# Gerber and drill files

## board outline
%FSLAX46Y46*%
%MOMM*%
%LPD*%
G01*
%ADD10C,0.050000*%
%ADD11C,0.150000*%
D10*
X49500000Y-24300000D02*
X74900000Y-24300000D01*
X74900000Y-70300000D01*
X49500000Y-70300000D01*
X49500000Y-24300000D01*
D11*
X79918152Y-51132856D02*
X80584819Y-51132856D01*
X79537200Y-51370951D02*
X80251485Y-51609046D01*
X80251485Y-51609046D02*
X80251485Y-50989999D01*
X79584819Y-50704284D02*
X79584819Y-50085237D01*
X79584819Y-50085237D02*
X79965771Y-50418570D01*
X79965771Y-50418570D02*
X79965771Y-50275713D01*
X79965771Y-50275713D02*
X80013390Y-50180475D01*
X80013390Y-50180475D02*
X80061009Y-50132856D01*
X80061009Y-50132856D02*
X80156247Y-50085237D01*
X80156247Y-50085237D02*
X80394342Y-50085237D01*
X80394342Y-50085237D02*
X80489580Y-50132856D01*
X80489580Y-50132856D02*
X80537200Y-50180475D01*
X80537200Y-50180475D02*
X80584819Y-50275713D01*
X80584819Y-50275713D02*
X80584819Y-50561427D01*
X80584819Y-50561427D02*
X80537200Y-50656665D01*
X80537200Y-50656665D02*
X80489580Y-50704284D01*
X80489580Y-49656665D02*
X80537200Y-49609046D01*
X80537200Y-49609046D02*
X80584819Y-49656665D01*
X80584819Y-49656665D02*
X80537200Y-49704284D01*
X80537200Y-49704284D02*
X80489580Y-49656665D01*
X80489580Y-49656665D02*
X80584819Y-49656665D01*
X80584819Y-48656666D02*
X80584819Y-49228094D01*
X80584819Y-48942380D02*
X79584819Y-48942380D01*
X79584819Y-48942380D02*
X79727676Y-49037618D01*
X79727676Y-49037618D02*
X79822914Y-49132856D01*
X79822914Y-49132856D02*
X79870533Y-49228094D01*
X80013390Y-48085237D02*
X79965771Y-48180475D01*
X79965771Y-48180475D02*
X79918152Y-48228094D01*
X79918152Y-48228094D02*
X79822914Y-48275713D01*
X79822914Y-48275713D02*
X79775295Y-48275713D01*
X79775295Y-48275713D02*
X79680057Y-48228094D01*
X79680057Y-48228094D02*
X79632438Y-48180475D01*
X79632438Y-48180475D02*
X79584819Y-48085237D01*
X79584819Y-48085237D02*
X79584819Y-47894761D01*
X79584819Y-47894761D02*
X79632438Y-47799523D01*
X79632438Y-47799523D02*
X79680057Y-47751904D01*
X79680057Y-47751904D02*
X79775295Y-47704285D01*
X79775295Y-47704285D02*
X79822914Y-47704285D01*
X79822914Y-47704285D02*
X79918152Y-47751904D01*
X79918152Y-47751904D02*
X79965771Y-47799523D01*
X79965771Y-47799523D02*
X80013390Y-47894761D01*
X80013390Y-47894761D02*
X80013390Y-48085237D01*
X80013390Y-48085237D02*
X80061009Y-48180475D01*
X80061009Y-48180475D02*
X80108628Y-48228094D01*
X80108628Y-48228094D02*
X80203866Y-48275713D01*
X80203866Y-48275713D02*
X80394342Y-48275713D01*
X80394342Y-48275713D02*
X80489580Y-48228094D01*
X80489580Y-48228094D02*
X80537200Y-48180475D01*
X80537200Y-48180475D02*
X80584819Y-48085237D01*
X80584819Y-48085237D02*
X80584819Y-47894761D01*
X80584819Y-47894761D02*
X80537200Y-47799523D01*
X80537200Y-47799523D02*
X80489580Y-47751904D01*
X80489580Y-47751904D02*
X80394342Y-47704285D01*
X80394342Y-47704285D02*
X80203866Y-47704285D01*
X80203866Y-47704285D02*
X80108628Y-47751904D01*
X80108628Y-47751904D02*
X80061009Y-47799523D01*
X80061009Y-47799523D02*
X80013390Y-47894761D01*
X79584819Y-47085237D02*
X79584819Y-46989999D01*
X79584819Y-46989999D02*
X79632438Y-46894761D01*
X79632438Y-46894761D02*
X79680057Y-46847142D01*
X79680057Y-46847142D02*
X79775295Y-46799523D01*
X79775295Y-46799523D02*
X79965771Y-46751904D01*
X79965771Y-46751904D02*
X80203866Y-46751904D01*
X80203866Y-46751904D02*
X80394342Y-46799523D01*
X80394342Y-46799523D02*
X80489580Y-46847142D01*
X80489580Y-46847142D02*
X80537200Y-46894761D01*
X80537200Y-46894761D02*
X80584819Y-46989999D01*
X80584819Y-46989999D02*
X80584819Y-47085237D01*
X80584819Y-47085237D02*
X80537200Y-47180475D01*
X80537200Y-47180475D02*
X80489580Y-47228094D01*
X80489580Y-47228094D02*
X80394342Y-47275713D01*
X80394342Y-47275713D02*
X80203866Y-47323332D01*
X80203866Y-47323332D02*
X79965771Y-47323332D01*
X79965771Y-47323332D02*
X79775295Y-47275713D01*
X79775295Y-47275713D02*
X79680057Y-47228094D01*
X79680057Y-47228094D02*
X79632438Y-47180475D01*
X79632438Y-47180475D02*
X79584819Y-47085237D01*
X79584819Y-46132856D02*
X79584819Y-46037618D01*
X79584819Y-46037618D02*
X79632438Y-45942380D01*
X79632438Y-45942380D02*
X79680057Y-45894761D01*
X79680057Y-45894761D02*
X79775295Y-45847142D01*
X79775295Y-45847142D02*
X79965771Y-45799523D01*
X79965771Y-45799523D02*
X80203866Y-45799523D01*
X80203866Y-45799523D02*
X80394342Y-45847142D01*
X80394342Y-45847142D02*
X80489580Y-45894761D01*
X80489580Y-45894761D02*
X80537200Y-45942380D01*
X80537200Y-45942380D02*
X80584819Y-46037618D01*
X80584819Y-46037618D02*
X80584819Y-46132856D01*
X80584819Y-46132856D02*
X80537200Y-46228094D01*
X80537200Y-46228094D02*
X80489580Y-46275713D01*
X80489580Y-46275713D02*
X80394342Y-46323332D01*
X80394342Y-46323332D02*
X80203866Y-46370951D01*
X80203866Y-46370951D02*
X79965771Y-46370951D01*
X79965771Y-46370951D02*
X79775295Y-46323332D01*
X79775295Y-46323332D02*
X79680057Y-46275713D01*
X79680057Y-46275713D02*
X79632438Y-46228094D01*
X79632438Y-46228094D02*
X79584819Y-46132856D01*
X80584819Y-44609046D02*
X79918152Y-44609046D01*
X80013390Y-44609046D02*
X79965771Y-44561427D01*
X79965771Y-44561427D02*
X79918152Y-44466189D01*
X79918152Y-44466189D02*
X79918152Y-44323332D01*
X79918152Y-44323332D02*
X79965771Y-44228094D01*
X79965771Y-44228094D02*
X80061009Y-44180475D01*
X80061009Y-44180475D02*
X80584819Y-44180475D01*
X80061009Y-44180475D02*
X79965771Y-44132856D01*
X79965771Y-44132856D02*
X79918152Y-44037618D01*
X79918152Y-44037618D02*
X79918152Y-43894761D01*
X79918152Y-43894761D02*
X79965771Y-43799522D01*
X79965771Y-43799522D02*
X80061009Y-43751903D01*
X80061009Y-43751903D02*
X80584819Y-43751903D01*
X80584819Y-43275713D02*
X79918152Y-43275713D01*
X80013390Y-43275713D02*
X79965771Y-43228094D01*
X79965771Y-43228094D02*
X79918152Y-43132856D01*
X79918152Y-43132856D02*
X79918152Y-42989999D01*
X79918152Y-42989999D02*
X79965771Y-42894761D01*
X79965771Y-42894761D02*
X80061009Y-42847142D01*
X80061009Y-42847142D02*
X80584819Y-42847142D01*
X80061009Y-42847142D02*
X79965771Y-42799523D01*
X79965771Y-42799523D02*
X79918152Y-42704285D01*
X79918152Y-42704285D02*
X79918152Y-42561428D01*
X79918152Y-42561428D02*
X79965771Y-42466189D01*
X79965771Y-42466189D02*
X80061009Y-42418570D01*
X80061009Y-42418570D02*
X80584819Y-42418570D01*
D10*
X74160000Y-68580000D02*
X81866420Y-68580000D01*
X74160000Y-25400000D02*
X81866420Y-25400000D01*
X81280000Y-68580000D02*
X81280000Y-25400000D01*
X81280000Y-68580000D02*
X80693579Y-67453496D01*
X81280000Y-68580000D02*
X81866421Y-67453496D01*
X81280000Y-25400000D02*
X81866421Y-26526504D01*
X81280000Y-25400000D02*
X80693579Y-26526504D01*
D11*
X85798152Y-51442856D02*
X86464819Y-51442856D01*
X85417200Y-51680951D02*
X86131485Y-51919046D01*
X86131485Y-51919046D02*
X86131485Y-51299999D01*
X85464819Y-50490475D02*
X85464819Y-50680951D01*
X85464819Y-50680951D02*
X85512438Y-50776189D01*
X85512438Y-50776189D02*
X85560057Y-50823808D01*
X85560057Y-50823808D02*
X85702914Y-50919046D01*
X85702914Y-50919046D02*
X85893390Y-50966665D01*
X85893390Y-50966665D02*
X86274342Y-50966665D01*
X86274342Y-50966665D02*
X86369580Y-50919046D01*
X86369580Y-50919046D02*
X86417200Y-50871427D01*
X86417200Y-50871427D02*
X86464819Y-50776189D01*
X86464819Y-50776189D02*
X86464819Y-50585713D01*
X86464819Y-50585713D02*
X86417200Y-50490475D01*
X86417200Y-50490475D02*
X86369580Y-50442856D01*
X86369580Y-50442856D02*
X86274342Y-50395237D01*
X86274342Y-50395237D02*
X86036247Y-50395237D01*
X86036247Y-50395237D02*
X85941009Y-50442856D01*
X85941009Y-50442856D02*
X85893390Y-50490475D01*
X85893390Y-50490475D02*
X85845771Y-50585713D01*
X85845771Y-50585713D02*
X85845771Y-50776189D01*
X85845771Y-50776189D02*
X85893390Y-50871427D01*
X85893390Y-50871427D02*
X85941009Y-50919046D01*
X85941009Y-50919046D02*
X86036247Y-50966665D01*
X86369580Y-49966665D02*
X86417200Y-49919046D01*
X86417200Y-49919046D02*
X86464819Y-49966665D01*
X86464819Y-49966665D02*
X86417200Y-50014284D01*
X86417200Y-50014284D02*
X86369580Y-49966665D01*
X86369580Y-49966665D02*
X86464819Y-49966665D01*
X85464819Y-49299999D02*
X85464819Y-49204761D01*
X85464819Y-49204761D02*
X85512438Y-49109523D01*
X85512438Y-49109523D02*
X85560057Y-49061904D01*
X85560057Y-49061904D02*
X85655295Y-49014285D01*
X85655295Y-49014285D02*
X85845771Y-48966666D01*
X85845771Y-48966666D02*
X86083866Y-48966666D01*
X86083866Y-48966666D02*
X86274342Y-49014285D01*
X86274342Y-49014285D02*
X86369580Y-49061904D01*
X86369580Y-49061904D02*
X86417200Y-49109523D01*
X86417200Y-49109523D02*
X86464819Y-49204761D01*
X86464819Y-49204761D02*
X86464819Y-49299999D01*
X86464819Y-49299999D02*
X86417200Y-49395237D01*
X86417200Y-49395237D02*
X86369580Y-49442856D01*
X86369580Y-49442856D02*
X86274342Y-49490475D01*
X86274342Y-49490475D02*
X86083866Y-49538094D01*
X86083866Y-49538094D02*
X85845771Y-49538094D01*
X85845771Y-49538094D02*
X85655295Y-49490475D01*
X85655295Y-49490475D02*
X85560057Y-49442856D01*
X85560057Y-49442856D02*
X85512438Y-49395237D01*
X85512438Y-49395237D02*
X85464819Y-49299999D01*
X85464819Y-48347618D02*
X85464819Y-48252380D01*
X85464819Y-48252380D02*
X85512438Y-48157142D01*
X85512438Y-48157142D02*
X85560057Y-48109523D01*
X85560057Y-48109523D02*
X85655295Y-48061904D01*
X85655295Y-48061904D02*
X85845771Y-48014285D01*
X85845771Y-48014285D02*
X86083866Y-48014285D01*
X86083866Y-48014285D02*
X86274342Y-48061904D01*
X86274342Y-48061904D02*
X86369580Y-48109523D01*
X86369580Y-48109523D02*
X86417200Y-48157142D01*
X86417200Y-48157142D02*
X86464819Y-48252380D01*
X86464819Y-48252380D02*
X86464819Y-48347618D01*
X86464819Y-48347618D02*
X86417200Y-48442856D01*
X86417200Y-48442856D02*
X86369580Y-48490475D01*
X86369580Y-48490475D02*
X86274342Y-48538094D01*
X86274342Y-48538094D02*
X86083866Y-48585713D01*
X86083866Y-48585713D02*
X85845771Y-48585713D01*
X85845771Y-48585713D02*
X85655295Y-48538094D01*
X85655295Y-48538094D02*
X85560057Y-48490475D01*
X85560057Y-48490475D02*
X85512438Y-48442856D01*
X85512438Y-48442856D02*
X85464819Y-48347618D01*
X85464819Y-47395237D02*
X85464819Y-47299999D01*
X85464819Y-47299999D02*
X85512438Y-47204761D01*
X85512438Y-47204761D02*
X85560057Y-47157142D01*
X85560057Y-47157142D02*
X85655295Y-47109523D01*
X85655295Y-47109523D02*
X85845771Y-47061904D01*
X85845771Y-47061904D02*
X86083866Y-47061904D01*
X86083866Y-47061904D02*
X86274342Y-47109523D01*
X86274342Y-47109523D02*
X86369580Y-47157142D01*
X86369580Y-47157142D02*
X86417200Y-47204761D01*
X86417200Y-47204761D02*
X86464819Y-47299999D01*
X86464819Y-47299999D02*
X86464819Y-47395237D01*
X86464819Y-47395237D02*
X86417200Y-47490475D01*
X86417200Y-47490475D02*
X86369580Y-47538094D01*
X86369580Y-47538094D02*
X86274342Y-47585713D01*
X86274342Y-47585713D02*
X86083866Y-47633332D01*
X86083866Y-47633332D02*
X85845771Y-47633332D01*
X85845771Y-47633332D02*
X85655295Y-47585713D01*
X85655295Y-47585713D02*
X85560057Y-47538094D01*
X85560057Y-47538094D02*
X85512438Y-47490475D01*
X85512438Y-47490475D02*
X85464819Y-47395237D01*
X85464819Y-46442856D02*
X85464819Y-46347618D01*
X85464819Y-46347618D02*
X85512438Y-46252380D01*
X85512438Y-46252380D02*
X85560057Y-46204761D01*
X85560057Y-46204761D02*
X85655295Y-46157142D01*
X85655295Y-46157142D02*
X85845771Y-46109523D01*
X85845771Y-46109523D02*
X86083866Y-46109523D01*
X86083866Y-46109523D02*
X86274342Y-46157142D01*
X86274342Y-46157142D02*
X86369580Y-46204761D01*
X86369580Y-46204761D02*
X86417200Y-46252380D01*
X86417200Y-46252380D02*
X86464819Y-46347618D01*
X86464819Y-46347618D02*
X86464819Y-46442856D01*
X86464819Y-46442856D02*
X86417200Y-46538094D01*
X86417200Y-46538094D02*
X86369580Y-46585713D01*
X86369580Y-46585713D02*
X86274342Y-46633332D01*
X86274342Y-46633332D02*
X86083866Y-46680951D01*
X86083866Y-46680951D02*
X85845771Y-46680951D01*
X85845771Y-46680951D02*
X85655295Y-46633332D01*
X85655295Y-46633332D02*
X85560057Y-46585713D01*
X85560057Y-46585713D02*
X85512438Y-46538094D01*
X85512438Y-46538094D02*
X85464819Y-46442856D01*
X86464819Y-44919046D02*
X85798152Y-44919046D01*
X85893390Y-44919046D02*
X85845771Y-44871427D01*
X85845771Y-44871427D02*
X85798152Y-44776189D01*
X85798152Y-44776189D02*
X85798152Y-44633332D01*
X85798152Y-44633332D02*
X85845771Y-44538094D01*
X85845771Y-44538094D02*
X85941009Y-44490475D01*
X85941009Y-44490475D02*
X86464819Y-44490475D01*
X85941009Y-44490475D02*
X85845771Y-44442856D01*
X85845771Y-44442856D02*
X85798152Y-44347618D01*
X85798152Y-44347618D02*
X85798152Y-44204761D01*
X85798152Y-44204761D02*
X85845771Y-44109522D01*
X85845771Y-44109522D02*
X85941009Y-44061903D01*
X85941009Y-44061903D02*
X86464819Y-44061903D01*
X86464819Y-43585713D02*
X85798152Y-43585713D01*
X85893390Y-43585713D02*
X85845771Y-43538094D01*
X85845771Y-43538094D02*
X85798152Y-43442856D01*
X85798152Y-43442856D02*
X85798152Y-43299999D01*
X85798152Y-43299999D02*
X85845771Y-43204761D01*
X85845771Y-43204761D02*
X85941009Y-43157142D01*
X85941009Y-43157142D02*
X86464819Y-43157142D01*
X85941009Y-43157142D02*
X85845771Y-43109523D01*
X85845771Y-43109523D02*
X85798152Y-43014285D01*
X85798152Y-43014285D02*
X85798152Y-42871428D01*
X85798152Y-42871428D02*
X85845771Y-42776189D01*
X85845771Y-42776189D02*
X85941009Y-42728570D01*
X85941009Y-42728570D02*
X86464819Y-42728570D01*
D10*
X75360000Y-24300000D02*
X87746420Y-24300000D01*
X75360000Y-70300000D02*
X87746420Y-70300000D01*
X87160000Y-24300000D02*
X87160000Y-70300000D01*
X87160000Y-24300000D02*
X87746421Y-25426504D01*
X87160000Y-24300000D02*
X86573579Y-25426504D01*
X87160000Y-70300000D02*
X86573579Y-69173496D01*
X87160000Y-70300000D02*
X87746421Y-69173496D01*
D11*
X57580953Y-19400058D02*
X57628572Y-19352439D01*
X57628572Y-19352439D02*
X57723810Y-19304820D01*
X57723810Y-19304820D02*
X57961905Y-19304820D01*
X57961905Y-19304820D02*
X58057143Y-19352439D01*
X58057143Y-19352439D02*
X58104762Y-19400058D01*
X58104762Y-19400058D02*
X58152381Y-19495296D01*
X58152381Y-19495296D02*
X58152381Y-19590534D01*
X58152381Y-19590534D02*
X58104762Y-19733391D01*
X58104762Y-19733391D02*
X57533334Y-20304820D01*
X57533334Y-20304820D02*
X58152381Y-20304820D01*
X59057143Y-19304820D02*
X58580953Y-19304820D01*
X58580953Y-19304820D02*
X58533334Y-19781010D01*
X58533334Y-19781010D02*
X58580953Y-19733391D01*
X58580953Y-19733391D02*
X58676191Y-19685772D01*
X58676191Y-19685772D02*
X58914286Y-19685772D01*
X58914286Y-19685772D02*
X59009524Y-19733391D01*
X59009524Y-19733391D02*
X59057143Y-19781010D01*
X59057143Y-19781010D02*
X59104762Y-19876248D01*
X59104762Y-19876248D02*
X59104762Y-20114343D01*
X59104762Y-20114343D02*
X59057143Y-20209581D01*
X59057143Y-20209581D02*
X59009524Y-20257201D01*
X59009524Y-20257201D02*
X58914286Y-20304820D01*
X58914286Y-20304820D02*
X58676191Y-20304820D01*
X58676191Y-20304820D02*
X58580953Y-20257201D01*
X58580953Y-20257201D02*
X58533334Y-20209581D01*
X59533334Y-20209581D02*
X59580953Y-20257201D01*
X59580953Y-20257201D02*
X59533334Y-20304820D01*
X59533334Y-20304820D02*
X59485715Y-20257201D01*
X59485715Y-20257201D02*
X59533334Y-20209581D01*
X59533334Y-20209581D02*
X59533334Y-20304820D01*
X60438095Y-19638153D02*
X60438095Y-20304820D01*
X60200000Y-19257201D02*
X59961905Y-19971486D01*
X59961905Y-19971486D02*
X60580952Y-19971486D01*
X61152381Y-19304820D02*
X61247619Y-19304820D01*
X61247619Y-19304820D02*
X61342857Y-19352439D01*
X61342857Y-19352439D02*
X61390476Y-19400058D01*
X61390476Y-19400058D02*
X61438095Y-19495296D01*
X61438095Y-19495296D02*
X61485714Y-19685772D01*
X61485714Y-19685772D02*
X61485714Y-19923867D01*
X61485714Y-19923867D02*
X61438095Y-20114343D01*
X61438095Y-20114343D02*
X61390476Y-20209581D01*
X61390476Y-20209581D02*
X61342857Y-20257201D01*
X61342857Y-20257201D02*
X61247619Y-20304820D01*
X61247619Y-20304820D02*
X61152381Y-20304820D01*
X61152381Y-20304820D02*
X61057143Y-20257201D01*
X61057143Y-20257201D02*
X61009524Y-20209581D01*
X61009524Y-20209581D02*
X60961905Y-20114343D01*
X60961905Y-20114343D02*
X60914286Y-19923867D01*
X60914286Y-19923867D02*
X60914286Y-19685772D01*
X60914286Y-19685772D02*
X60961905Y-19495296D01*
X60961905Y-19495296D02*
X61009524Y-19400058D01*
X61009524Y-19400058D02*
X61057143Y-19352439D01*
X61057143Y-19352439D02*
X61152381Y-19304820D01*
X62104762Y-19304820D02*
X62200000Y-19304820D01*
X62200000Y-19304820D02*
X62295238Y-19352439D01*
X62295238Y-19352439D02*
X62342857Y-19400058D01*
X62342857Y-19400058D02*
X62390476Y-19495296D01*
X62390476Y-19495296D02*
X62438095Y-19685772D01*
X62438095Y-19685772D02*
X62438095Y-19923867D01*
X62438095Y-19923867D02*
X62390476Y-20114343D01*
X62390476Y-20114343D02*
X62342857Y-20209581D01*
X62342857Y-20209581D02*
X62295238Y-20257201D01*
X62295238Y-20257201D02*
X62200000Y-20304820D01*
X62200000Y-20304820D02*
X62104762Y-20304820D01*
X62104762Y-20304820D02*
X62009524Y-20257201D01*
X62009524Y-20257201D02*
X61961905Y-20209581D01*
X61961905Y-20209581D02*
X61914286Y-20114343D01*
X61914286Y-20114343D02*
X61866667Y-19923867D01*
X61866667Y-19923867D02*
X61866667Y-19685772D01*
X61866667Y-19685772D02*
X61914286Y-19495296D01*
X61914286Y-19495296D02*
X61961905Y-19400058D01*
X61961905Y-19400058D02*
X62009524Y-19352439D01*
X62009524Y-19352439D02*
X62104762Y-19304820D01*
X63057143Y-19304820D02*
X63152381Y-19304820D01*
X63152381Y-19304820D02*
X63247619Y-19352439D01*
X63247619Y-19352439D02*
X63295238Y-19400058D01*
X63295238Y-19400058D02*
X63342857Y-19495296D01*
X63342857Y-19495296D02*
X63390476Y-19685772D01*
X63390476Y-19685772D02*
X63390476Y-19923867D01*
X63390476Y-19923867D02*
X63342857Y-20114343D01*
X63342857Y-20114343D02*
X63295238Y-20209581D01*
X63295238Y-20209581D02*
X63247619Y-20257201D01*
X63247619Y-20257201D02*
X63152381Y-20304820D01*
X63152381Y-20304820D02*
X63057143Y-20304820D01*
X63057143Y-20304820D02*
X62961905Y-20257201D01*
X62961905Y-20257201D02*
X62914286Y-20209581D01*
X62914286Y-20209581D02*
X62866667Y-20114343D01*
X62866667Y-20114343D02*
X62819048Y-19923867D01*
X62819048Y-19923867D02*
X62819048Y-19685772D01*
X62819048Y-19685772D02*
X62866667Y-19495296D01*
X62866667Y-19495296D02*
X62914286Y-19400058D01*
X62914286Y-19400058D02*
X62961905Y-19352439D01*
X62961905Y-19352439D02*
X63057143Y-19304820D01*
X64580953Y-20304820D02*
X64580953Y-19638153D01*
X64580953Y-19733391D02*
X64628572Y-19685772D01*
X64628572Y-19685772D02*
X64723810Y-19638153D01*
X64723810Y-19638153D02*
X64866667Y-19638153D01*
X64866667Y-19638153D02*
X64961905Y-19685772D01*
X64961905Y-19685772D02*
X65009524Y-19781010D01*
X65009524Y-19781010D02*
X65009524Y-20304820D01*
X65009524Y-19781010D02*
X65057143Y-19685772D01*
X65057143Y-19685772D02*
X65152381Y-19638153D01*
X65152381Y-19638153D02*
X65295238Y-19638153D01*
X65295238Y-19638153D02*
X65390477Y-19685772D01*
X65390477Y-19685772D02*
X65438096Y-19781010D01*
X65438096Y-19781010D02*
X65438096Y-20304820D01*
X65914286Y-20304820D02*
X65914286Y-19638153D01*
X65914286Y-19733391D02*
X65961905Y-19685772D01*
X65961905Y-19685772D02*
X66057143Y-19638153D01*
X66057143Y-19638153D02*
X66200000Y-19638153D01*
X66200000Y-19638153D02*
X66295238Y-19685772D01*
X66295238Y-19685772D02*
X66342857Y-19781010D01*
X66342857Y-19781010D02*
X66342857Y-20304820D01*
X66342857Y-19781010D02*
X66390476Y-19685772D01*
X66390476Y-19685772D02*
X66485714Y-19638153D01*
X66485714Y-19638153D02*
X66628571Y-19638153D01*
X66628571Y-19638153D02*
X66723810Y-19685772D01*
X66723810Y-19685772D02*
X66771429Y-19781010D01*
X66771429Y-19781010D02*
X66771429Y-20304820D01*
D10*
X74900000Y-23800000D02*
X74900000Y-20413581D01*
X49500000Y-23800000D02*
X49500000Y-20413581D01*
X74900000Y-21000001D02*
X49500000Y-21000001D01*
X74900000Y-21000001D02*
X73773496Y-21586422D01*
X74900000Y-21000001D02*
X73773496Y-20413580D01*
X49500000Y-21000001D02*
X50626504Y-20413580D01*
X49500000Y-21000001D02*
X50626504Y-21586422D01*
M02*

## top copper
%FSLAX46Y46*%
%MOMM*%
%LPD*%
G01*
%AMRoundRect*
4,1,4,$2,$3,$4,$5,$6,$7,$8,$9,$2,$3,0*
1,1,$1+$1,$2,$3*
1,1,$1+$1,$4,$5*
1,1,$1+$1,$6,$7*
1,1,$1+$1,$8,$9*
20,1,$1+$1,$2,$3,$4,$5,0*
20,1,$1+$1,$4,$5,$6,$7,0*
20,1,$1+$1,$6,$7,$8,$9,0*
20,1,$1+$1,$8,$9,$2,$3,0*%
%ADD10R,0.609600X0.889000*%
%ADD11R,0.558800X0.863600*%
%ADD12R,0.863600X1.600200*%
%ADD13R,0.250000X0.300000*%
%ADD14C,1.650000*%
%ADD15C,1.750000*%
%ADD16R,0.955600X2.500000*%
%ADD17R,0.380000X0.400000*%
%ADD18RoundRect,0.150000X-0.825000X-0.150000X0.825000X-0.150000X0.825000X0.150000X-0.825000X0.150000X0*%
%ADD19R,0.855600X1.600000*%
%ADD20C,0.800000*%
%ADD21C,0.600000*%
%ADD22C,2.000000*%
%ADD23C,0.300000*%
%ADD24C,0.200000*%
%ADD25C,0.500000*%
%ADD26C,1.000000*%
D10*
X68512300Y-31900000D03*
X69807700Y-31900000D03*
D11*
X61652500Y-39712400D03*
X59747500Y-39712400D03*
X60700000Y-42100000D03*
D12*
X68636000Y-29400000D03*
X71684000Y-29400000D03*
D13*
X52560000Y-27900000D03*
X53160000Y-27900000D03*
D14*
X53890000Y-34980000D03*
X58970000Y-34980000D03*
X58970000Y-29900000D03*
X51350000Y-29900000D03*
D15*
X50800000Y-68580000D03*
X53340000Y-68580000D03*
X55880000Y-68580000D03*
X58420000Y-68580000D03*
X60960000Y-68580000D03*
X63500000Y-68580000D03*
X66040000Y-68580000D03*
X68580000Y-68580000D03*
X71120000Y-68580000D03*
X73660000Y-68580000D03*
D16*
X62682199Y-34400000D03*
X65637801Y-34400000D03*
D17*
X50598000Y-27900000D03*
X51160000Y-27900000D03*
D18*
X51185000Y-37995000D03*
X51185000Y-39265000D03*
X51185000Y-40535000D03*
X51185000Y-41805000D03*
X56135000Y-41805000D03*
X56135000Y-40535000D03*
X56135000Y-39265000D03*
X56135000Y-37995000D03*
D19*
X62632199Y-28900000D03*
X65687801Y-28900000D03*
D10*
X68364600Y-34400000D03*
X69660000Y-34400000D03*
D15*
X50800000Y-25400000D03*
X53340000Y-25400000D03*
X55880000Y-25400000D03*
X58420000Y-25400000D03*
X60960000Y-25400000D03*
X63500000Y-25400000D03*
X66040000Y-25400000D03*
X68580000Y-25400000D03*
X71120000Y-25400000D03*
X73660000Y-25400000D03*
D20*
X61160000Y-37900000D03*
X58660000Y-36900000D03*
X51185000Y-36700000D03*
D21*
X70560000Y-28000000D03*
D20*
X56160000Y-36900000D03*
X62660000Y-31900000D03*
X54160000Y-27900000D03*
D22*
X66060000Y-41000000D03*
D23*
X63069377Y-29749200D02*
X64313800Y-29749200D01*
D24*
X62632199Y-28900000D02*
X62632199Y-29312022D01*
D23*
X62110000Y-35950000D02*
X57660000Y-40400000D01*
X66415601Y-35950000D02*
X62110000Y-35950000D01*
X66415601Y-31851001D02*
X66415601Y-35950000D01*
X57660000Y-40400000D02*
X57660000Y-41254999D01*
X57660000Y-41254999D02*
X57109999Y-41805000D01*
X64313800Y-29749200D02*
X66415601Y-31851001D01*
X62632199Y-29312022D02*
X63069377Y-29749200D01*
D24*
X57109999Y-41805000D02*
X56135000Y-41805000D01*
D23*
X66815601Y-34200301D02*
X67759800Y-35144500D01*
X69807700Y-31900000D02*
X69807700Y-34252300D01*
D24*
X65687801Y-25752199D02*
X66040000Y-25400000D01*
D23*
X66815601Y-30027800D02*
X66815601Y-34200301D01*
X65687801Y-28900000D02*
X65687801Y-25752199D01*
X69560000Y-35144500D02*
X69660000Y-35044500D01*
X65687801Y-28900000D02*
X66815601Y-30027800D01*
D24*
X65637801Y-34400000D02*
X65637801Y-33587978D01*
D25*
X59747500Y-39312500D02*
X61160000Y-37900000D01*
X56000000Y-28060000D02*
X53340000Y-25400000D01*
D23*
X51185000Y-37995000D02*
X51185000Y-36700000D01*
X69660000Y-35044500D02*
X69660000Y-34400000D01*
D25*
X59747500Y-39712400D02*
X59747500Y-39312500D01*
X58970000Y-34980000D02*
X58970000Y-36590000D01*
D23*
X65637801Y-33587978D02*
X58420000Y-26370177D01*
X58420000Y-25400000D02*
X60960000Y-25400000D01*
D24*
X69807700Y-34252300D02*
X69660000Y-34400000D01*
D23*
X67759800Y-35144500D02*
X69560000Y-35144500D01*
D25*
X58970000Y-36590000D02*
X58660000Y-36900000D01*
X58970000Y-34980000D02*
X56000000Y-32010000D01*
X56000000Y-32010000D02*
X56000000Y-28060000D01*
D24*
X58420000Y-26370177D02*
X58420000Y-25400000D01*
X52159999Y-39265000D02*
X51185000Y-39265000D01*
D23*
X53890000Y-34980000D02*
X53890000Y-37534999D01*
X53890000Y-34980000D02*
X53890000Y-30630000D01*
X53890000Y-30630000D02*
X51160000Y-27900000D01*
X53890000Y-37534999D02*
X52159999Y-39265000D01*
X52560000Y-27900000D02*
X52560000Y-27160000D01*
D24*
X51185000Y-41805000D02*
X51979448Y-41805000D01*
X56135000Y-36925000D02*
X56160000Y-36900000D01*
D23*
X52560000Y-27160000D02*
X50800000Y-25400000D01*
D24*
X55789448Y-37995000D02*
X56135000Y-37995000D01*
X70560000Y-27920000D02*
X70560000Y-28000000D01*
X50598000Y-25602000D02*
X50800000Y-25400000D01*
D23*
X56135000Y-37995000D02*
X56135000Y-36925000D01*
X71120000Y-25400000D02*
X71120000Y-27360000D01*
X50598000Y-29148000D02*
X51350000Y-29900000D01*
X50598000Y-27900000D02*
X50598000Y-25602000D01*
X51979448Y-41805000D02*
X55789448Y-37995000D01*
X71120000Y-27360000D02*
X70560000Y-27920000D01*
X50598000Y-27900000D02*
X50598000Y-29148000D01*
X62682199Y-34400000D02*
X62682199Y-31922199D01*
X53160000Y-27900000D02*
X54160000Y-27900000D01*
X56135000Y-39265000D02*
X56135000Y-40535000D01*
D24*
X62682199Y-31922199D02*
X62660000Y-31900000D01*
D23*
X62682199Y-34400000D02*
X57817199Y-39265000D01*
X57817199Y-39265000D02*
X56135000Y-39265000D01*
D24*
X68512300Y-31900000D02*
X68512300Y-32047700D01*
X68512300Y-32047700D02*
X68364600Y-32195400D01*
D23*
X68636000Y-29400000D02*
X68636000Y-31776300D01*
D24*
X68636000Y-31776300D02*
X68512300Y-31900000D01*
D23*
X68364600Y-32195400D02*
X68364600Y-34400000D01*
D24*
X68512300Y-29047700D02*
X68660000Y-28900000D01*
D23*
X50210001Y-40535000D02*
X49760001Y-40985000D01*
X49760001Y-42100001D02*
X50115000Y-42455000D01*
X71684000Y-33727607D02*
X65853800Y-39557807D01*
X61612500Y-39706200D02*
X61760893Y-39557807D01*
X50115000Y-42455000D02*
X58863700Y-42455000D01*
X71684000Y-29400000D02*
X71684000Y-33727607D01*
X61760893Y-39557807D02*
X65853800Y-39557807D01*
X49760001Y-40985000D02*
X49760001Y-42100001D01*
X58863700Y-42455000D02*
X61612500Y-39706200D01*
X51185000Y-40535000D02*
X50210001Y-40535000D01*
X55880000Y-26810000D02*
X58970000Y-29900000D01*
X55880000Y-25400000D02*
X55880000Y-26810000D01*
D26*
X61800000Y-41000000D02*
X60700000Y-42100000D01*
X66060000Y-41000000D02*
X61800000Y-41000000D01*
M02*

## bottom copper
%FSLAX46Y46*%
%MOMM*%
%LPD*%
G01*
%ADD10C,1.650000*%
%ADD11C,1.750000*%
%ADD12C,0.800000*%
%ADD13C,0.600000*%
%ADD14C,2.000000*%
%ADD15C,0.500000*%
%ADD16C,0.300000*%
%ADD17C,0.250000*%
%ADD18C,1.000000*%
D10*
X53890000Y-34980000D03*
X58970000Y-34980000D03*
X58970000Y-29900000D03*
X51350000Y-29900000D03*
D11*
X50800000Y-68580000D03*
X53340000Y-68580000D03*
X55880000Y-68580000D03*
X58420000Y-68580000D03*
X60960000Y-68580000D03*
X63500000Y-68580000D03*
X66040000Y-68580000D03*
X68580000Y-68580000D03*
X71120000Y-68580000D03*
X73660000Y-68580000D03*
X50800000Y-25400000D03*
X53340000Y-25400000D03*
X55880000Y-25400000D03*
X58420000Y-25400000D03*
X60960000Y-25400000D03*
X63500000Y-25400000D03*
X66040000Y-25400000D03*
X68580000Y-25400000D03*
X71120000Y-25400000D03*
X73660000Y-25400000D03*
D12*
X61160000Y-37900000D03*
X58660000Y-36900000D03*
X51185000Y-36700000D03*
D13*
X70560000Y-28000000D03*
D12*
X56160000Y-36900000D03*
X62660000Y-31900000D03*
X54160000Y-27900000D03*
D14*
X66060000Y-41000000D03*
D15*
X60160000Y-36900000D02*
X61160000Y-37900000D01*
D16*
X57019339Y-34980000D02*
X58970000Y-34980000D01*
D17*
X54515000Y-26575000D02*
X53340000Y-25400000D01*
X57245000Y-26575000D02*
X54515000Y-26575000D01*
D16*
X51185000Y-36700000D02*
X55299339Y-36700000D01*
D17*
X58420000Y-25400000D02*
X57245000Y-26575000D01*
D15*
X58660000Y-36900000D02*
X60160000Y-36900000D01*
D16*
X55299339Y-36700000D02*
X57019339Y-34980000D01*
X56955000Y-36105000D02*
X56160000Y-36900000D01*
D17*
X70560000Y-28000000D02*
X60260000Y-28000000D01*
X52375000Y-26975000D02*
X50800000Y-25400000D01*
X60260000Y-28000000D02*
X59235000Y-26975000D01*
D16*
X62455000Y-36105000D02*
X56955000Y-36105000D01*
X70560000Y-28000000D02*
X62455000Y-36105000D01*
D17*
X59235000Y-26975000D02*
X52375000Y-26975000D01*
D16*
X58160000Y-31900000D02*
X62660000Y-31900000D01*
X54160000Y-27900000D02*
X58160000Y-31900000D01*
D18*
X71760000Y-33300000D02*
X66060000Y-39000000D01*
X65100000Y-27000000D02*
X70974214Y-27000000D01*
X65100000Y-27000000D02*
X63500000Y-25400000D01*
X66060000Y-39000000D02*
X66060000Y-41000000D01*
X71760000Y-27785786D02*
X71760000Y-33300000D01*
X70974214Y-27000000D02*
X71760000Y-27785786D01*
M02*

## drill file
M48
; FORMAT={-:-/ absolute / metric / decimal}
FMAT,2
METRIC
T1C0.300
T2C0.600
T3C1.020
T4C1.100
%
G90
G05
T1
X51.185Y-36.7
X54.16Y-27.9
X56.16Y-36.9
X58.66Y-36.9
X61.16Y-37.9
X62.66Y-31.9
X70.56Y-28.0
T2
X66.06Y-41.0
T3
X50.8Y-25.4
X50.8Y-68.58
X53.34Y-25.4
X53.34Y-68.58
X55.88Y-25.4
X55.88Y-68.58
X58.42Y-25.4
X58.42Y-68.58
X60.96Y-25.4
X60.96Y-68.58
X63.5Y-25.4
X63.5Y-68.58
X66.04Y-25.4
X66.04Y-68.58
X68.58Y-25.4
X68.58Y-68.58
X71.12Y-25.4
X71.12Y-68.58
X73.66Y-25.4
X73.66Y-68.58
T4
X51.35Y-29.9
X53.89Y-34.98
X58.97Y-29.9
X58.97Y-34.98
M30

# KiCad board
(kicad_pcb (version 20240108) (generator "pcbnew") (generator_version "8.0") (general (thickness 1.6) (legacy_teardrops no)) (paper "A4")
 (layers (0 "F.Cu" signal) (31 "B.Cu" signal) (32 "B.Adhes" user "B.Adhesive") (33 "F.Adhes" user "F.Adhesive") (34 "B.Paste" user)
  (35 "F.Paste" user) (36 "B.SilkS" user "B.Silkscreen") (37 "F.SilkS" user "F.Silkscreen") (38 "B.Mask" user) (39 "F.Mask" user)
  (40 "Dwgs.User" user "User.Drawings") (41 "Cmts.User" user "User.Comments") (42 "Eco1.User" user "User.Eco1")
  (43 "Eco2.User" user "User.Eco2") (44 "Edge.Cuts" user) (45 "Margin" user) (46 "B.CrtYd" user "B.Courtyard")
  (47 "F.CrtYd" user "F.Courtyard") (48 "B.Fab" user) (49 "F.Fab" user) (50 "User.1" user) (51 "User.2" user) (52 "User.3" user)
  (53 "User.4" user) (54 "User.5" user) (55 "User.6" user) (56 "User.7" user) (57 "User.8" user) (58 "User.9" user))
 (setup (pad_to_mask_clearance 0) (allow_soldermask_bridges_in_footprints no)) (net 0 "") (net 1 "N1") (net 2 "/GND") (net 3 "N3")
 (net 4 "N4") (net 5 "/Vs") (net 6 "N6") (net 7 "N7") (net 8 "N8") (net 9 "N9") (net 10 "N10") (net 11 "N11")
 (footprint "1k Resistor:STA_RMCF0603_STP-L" (layer "F.Cu") (at 69.16 31.9)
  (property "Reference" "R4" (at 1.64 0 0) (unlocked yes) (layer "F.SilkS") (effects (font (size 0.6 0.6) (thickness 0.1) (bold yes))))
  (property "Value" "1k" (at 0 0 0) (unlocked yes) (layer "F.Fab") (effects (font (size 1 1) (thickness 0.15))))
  (pad "1" smd rect (at -0.6477 0) (size 0.6096 0.889) (layers "F.Cu" "F.Paste" "F.Mask") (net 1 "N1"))
  (pad "2" smd rect (at 0.6477 0) (size 0.6096 0.889) (layers "F.Cu" "F.Paste" "F.Mask") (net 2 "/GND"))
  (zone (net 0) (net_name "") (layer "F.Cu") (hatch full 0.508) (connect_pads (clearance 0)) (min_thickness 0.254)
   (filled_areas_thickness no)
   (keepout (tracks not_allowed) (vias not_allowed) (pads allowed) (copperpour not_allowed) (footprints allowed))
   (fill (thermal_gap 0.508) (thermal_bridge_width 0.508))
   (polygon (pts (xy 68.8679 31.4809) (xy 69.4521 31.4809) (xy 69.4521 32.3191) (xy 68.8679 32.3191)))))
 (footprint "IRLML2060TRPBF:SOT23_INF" (layer "F.Cu") (at 60.7 40.9062 180)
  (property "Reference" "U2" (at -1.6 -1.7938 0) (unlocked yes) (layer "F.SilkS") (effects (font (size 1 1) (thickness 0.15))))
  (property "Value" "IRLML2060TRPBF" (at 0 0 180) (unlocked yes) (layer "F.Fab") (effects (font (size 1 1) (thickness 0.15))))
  (pad "1" smd rect (at -0.9525 1.1938 180) (size 0.5588 0.8636) (layers "F.Cu" "F.Paste" "F.Mask") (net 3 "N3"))
  (pad "2" smd rect (at 0.9525 1.1938 180) (size 0.5588 0.8636) (layers "F.Cu" "F.Paste" "F.Mask") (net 2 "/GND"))
  (pad "3" smd rect (at 0 -1.1938 180) (size 0.5588 0.8636) (layers "F.Cu" "F.Paste" "F.Mask") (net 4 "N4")))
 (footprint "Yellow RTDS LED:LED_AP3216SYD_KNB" (layer "F.Cu") (at 70.16 29.4)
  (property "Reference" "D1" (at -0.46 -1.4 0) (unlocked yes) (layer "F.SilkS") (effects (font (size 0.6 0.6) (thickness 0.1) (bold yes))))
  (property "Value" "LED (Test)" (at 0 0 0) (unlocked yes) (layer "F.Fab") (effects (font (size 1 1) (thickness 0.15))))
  (pad "1" smd rect (at -1.524 0) (size 0.8636 1.6002) (layers "F.Cu" "F.Paste" "F.Mask") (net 1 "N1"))
  (pad "2" smd rect (at 1.524 0) (size 0.8636 1.6002) (layers "F.Cu" "F.Paste" "F.Mask") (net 3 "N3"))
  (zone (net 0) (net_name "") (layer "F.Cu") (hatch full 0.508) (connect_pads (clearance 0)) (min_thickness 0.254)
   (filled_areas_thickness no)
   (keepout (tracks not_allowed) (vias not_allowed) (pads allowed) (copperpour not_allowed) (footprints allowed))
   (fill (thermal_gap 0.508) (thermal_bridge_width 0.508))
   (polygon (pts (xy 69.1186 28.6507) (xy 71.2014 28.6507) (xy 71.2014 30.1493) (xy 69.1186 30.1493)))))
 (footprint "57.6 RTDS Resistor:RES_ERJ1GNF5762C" (layer "F.Cu") (at 52.86 27.9)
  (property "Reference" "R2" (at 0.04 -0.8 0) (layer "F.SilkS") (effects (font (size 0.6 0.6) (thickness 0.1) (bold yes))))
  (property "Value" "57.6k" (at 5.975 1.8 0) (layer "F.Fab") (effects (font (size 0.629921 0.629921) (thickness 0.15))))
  (pad "1" smd rect (at -0.3 0) (size 0.25 0.3) (layers "F.Cu" "F.Paste" "F.Mask") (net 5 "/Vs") (solder_mask_margin 0.102))
  (pad "2" smd rect (at 0.3 0) (size 0.25 0.3) (layers "F.Cu" "F.Paste" "F.Mask") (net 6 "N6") (solder_mask_margin 0.102)))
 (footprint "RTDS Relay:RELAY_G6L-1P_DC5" (layer "F.Cu") (at 55.16 32.44)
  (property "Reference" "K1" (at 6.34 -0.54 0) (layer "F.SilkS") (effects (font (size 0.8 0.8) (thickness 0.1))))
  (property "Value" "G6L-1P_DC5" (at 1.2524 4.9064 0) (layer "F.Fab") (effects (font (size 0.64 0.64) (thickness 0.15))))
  (pad "2" thru_hole circle (at -1.27 2.54) (size 1.65 1.65) (drill 1.1) (layers "*.Cu" "*.Mask") (remove_unused_layers no) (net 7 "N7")
   (solder_mask_margin 0.102))
  (pad "4" thru_hole circle (at 3.81 2.54) (size 1.65 1.65) (drill 1.1) (layers "*.Cu" "*.Mask") (remove_unused_layers no) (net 2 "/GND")
   (solder_mask_margin 0.102))
  (pad "5" thru_hole circle (at 3.81 -2.54) (size 1.65 1.65) (drill 1.1) (layers "*.Cu" "*.Mask") (remove_unused_layers no) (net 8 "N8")
   (solder_mask_margin 0.102))
  (pad "8" thru_hole circle (at -3.81 -2.54) (size 1.65 1.65) (drill 1.1) (layers "*.Cu" "*.Mask") (remove_unused_layers no) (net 5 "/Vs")
   (solder_mask_margin 0.102)))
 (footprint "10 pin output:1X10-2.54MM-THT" (layer "F.Cu") (at 50.8 68.58)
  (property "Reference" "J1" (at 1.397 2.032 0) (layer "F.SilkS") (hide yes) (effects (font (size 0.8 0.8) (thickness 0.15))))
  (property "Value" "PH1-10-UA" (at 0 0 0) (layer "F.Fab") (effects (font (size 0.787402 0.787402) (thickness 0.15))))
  (pad "1" thru_hole circle (at 0 0) (size 1.75 1.75) (drill 1.02) (layers "*.Cu" "*.Mask") (remove_unused_layers no)
   (solder_mask_margin 0.102))
  (pad "2" thru_hole circle (at 2.54 0) (size 1.75 1.75) (drill 1.02) (layers "*.Cu" "*.Mask") (remove_unused_layers no)
   (solder_mask_margin 0.102))
  (pad "3" thru_hole circle (at 5.08 0) (size 1.75 1.75) (drill 1.02) (layers "*.Cu" "*.Mask") (remove_unused_layers no)
   (solder_mask_margin 0.102))
  (pad "4" thru_hole circle (at 7.62 0) (size 1.75 1.75) (drill 1.02) (layers "*.Cu" "*.Mask") (remove_unused_layers no)
   (solder_mask_margin 0.102))
  (pad "5" thru_hole circle (at 10.16 0) (size 1.75 1.75) (drill 1.02) (layers "*.Cu" "*.Mask") (remove_unused_layers no)
   (solder_mask_margin 0.102))
  (pad "6" thru_hole circle (at 12.7 0) (size 1.75 1.75) (drill 1.02) (layers "*.Cu" "*.Mask") (remove_unused_layers no)
   (solder_mask_margin 0.102))
  (pad "7" thru_hole circle (at 15.24 0) (size 1.75 1.75) (drill 1.02) (layers "*.Cu" "*.Mask") (remove_unused_layers no)
   (solder_mask_margin 0.102))
  (pad "8" thru_hole circle (at 17.78 0) (size 1.75 1.75) (drill 1.02) (layers "*.Cu" "*.Mask") (remove_unused_layers no)
   (solder_mask_margin 0.102))
  (pad "9" thru_hole circle (at 20.32 0) (size 1.75 1.75) (drill 1.02) (layers "*.Cu" "*.Mask") (remove_unused_layers no)
   (solder_mask_margin 0.102))
  (pad "10" thru_hole circle (at 22.86 0) (size 1.75 1.75) (drill 1.02) (layers "*.Cu" "*.Mask") (remove_unused_layers no)
   (solder_mask_margin 0.102)))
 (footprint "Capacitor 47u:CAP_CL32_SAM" (layer "F.Cu") (at 64.16 34.4)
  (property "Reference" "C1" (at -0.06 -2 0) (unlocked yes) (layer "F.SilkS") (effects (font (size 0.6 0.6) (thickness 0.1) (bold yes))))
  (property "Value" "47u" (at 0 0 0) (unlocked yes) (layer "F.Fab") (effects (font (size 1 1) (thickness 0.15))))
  (pad "1" smd rect (at -1.477801 0) (size 0.9556 2.5) (layers "F.Cu" "F.Paste" "F.Mask") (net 6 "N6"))
  (pad "2" smd rect (at 1.477801 0) (size 0.9556 2.5) (layers "F.Cu" "F.Paste" "F.Mask") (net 2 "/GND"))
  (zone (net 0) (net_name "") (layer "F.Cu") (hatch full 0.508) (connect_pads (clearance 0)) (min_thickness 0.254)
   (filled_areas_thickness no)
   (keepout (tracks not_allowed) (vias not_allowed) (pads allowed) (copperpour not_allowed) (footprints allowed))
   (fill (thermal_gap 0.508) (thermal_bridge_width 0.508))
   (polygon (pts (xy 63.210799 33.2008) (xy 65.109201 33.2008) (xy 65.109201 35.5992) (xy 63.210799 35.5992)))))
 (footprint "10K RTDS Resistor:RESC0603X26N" (layer "F.Cu") (at 50.879 27.9)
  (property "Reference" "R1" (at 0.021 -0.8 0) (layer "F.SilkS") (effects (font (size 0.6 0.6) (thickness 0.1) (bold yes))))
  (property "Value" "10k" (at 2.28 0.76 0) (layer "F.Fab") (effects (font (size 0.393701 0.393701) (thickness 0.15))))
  (pad "1" smd rect (at -0.281 0) (size 0.38 0.4) (layers "F.Cu" "F.Paste" "F.Mask") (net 5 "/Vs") (solder_mask_margin 0.102))
  (pad "2" smd rect (at 0.281 0) (size 0.38 0.4) (layers "F.Cu" "F.Paste" "F.Mask") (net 7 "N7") (solder_mask_margin 0.102)))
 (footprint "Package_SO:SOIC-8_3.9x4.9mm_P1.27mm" (layer "F.Cu") (at 53.66 39.9)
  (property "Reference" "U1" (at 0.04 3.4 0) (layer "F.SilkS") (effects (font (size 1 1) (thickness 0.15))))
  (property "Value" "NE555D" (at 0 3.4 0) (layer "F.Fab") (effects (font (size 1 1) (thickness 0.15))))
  (pad "1" smd roundrect (at -2.475 -1.905) (size 1.95 0.6) (layers "F.Cu" "F.Paste" "F.Mask") (roundrect_rratio 0.25) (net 2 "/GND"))
  (pad "2" smd roundrect (at -2.475 -0.635) (size 1.95 0.6) (layers "F.Cu" "F.Paste" "F.Mask") (roundrect_rratio 0.25) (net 7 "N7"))
  (pad "3" smd roundrect (at -2.475 0.635) (size 1.95 0.6) (layers "F.Cu" "F.Paste" "F.Mask") (roundrect_rratio 0.25) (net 3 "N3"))
  (pad "4" smd roundrect (at -2.475 1.905) (size 1.95 0.6) (layers "F.Cu" "F.Paste" "F.Mask") (roundrect_rratio 0.25) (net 5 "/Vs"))
  (pad "5" smd roundrect (at 2.475 1.905) (size 1.95 0.6) (layers "F.Cu" "F.Paste" "F.Mask") (roundrect_rratio 0.25) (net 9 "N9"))
  (pad "6" smd roundrect (at 2.475 0.635) (size 1.95 0.6) (layers "F.Cu" "F.Paste" "F.Mask") (roundrect_rratio 0.25) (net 6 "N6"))
  (pad "7" smd roundrect (at 2.475 -0.635) (size 1.95 0.6) (layers "F.Cu" "F.Paste" "F.Mask") (roundrect_rratio 0.25) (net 6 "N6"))
  (pad "8" smd roundrect (at 2.475 -1.905) (size 1.95 0.6) (layers "F.Cu" "F.Paste" "F.Mask") (roundrect_rratio 0.25) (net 5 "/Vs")))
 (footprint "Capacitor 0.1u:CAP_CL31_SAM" (layer "F.Cu") (at 64.16 28.9)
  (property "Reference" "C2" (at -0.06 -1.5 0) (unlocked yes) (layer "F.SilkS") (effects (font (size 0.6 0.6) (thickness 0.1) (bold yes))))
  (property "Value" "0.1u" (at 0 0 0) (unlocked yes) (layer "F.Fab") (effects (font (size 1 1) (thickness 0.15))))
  (pad "1" smd rect (at -1.527801 0) (size 0.8556 1.6) (layers "F.Cu" "F.Paste" "F.Mask") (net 9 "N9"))
  (pad "2" smd rect (at 1.527801 0) (size 0.8556 1.6) (layers "F.Cu" "F.Paste" "F.Mask") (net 2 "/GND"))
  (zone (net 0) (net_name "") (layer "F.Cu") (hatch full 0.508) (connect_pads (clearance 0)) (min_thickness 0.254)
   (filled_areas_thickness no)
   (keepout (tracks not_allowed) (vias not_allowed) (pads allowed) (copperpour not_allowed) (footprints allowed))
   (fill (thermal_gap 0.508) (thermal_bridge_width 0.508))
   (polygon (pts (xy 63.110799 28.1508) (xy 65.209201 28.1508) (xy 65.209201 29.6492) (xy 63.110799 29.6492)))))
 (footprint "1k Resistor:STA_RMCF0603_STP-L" (layer "F.Cu") (at 69.0123 34.4)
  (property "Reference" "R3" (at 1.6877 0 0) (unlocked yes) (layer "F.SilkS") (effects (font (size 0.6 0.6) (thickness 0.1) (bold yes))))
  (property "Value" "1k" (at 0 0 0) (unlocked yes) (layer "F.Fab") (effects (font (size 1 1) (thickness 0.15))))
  (pad "1" smd rect (at -0.6477 0) (size 0.6096 0.889) (layers "F.Cu" "F.Paste" "F.Mask") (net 1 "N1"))
  (pad "2" smd rect (at 0.6477 0) (size 0.6096 0.889) (layers "F.Cu" "F.Paste" "F.Mask") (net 2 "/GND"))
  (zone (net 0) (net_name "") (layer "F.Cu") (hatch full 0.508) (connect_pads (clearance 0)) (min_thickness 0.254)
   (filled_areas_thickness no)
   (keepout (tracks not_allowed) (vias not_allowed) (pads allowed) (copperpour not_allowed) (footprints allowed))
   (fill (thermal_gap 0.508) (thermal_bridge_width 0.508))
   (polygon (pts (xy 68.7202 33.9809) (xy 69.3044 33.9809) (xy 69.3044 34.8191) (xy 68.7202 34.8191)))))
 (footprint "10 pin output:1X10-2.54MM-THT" (layer "F.Cu") (at 50.8 25.4)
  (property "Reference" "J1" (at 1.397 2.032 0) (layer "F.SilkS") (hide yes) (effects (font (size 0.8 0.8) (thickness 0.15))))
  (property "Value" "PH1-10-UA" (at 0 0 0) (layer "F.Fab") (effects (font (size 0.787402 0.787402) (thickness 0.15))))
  (pad "1" thru_hole circle (at 0 0) (size 1.75 1.75) (drill 1.02) (layers "*.Cu" "*.Mask") (remove_unused_layers no) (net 5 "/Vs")
   (solder_mask_margin 0.102))
  (pad "2" thru_hole circle (at 2.54 0) (size 1.75 1.75) (drill 1.02) (layers "*.Cu" "*.Mask") (remove_unused_layers no) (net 2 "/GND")
   (solder_mask_margin 0.102))
  (pad "3" thru_hole circle (at 5.08 0) (size 1.75 1.75) (drill 1.02) (layers "*.Cu" "*.Mask") (remove_unused_layers no) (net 8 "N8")
   (solder_mask_margin 0.102))
  (pad "4" thru_hole circle (at 7.62 0) (size 1.75 1.75) (drill 1.02) (layers "*.Cu" "*.Mask") (remove_unused_layers no) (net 2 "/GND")
   (solder_mask_margin 0.102))
  (pad "5" thru_hole circle (at 10.16 0) (size 1.75 1.75) (drill 1.02) (layers "*.Cu" "*.Mask") (remove_unused_layers no) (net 2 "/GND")
   (solder_mask_margin 0.102))
  (pad "6" thru_hole circle (at 12.7 0) (size 1.75 1.75) (drill 1.02) (layers "*.Cu" "*.Mask") (remove_unused_layers no) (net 4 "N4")
   (solder_mask_margin 0.102))
  (pad "7" thru_hole circle (at 15.24 0) (size 1.75 1.75) (drill 1.02) (layers "*.Cu" "*.Mask") (remove_unused_layers no) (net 2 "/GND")
   (solder_mask_margin 0.102))
  (pad "8" thru_hole circle (at 17.78 0) (size 1.75 1.75) (drill 1.02) (layers "*.Cu" "*.Mask") (remove_unused_layers no) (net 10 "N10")
   (solder_mask_margin 0.102))
  (pad "9" thru_hole circle (at 20.32 0) (size 1.75 1.75) (drill 1.02) (layers "*.Cu" "*.Mask") (remove_unused_layers no) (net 5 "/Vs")
   (solder_mask_margin 0.102))
  (pad "10" thru_hole circle (at 22.86 0) (size 1.75 1.75) (drill 1.02) (layers "*.Cu" "*.Mask") (remove_unused_layers no) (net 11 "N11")
   (solder_mask_margin 0.102)))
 (gr_rect (start 49.5 24.3) (end 74.9 70.3) (stroke (width 0.05) (type default)) (fill none) (layer "Edge.Cuts"))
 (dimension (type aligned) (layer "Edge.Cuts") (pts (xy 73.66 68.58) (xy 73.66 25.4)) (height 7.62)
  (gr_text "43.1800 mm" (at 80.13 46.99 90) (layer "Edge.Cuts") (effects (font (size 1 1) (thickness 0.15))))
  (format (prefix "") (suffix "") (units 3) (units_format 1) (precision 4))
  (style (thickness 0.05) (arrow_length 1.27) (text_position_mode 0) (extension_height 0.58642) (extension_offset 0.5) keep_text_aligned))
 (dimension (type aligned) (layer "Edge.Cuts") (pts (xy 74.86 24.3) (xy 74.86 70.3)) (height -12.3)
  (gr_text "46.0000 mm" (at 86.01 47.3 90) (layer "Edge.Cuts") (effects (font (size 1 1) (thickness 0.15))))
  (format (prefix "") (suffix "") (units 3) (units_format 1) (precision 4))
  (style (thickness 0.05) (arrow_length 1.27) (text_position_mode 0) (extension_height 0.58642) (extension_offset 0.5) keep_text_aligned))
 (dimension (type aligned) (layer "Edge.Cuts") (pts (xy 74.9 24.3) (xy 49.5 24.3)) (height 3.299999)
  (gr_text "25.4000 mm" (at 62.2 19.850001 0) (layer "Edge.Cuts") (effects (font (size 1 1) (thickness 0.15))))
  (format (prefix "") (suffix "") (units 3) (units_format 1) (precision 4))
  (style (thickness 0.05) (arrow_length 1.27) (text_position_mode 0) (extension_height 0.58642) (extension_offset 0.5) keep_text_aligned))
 (segment (start 63.069377 29.7492) (end 64.3138 29.7492) (width 0.3) (layer "F.Cu") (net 9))
 (segment (start 62.632199 28.9) (end 62.632199 29.312022) (width 0.2) (layer "F.Cu") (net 9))
 (segment (start 62.11 35.95) (end 57.66 40.4) (width 0.3) (layer "F.Cu") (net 9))
 (segment (start 66.415601 35.95) (end 62.11 35.95) (width 0.3) (layer "F.Cu") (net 9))
 (segment (start 66.415601 31.851001) (end 66.415601 35.95) (width 0.3) (layer "F.Cu") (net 9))
 (segment (start 57.66 40.4) (end 57.66 41.254999) (width 0.3) (layer "F.Cu") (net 9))
 (segment (start 57.66 41.254999) (end 57.109999 41.805) (width 0.3) (layer "F.Cu") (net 9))
 (segment (start 64.3138 29.7492) (end 66.415601 31.851001) (width 0.3) (layer "F.Cu") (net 9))
 (segment (start 62.632199 29.312022) (end 63.069377 29.7492) (width 0.3) (layer "F.Cu") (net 9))
 (segment (start 57.109999 41.805) (end 56.135 41.805) (width 0.2) (layer "F.Cu") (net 9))
 (segment (start 66.815601 34.200301) (end 67.7598 35.1445) (width 0.3) (layer "F.Cu") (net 2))
 (segment (start 69.8077 31.9) (end 69.8077 34.2523) (width 0.3) (layer "F.Cu") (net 2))
 (segment (start 65.687801 25.752199) (end 66.04 25.4) (width 0.2) (layer "F.Cu") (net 2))
 (segment (start 66.815601 30.0278) (end 66.815601 34.200301) (width 0.3) (layer "F.Cu") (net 2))
 (segment (start 65.687801 28.9) (end 65.687801 25.752199) (width 0.3) (layer "F.Cu") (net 2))
 (segment (start 69.56 35.1445) (end 69.66 35.0445) (width 0.3) (layer "F.Cu") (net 2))
 (segment (start 65.687801 28.9) (end 66.815601 30.0278) (width 0.3) (layer "F.Cu") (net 2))
 (segment (start 65.637801 34.4) (end 65.637801 33.587978) (width 0.2) (layer "F.Cu") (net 2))
 (segment (start 59.7475 39.3125) (end 61.16 37.9) (width 0.5) (layer "F.Cu") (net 2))
 (segment (start 56 28.06) (end 53.34 25.4) (width 0.5) (layer "F.Cu") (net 2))
 (segment (start 51.185 37.995) (end 51.185 36.7) (width 0.3) (layer "F.Cu") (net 2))
 (segment (start 69.66 35.0445) (end 69.66 34.4) (width 0.3) (layer "F.Cu") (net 2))
 (segment (start 59.7475 39.7124) (end 59.7475 39.3125) (width 0.5) (layer "F.Cu") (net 2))
 (segment (start 58.97 34.98) (end 58.97 36.59) (width 0.5) (layer "F.Cu") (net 2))
 (segment (start 65.637801 33.587978) (end 58.42 26.370177) (width 0.3) (layer "F.Cu") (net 2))
 (segment (start 58.42 25.4) (end 60.96 25.4) (width 0.3) (layer "F.Cu") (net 2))
 (segment (start 69.8077 34.2523) (end 69.66 34.4) (width 0.2) (layer "F.Cu") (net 2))
 (segment (start 67.7598 35.1445) (end 69.56 35.1445) (width 0.3) (layer "F.Cu") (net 2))
 (segment (start 58.97 36.59) (end 58.66 36.9) (width 0.5) (layer "F.Cu") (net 2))
 (segment (start 58.97 34.98) (end 56 32.01) (width 0.5) (layer "F.Cu") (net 2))
 (segment (start 56 32.01) (end 56 28.06) (width 0.5) (layer "F.Cu") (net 2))
 (segment (start 58.42 26.370177) (end 58.42 25.4) (width 0.2) (layer "F.Cu") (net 2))
 (via (at 61.16 37.9) (size 0.8) (drill 0.3) (layers "F.Cu" "B.Cu") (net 2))
 (via (at 58.66 36.9) (size 0.8) (drill 0.3) (layers "F.Cu" "B.Cu") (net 2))
 (via (at 51.185 36.7) (size 0.8) (drill 0.3) (layers "F.Cu" "B.Cu") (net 2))
 (segment (start 60.16 36.9) (end 61.16 37.9) (width 0.5) (layer "B.Cu") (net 2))
 (segment (start 57.019339 34.98) (end 58.97 34.98) (width 0.3) (layer "B.Cu") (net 2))
 (segment (start 54.515 26.575) (end 53.34 25.4) (width 0.25) (layer "B.Cu") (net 2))
 (segment (start 57.245 26.575) (end 54.515 26.575) (width 0.25) (layer "B.Cu") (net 2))
 (segment (start 51.185 36.7) (end 55.299339 36.7) (width 0.3) (layer "B.Cu") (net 2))
 (segment (start 58.42 25.4) (end 57.245 26.575) (width 0.25) (layer "B.Cu") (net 2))
 (segment (start 58.66 36.9) (end 60.16 36.9) (width 0.5) (layer "B.Cu") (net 2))
 (segment (start 55.299339 36.7) (end 57.019339 34.98) (width 0.3) (layer "B.Cu") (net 2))
 (segment (start 52.159999 39.265) (end 51.185 39.265) (width 0.2) (layer "F.Cu") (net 7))
 (segment (start 53.89 34.98) (end 53.89 37.534999) (width 0.3) (layer "F.Cu") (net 7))
 (segment (start 53.89 34.98) (end 53.89 30.63) (width 0.3) (layer "F.Cu") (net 7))
 (segment (start 53.89 30.63) (end 51.16 27.9) (width 0.3) (layer "F.Cu") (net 7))
 (segment (start 53.89 37.534999) (end 52.159999 39.265) (width 0.3) (layer "F.Cu") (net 7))
 (segment (start 52.56 27.9) (end 52.56 27.16) (width 0.3) (layer "F.Cu") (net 5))
 (segment (start 51.185 41.805) (end 51.979448 41.805) (width 0.2) (layer "F.Cu") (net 5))
 (segment (start 56.135 36.925) (end 56.16 36.9) (width 0.2) (layer "F.Cu") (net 5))
 (segment (start 52.56 27.16) (end 50.8 25.4) (width 0.3) (layer "F.Cu") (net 5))
 (segment (start 55.789448 37.995) (end 56.135 37.995) (width 0.2) (layer "F.Cu") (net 5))
 (segment (start 70.56 27.92) (end 70.56 28) (width 0.2) (layer "F.Cu") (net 5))
 (segment (start 50.598 25.602) (end 50.8 25.4) (width 0.2) (layer "F.Cu") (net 5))
 (segment (start 56.135 37.995) (end 56.135 36.925) (width 0.3) (layer "F.Cu") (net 5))
 (segment (start 71.12 25.4) (end 71.12 27.36) (width 0.3) (layer "F.Cu") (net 5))
 (segment (start 50.598 29.148) (end 51.35 29.9) (width 0.3) (layer "F.Cu") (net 5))
 (segment (start 50.598 27.9) (end 50.598 25.602) (width 0.3) (layer "F.Cu") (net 5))
 (segment (start 51.979448 41.805) (end 55.789448 37.995) (width 0.3) (layer "F.Cu") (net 5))
 (segment (start 71.12 27.36) (end 70.56 27.92) (width 0.3) (layer "F.Cu") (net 5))
 (segment (start 50.598 27.9) (end 50.598 29.148) (width 0.3) (layer "F.Cu") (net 5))
 (via (at 70.56 28) (size 0.6) (drill 0.3) (layers "F.Cu" "B.Cu") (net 5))
 (via (at 56.16 36.9) (size 0.8) (drill 0.3) (layers "F.Cu" "B.Cu") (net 5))
 (segment (start 56.955 36.105) (end 56.16 36.9) (width 0.3) (layer "B.Cu") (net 5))
 (segment (start 70.56 28) (end 60.26 28) (width 0.25) (layer "B.Cu") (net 5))
 (segment (start 52.375 26.975) (end 50.8 25.4) (width 0.25) (layer "B.Cu") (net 5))
 (segment (start 60.26 28) (end 59.235 26.975) (width 0.25) (layer "B.Cu") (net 5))
 (segment (start 62.455 36.105) (end 56.955 36.105) (width 0.3) (layer "B.Cu") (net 5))
 (segment (start 70.56 28) (end 62.455 36.105) (width 0.3) (layer "B.Cu") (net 5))
 (segment (start 59.235 26.975) (end 52.375 26.975) (width 0.25) (layer "B.Cu") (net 5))
 (segment (start 62.682199 34.4) (end 62.682199 31.922199) (width 0.3) (layer "F.Cu") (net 6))
 (segment (start 53.16 27.9) (end 54.16 27.9) (width 0.3) (layer "F.Cu") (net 6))
 (segment (start 56.135 39.265) (end 56.135 40.535) (width 0.3) (layer "F.Cu") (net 6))
 (segment (start 62.682199 31.922199) (end 62.66 31.9) (width 0.2) (layer "F.Cu") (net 6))
 (segment (start 62.682199 34.4) (end 57.817199 39.265) (width 0.3) (layer "F.Cu") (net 6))
 (segment (start 57.817199 39.265) (end 56.135 39.265) (width 0.3) (layer "F.Cu") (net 6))
 (via (at 62.66 31.9) (size 0.8) (drill 0.3) (layers "F.Cu" "B.Cu") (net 6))
 (via (at 54.16 27.9) (size 0.8) (drill 0.3) (layers "F.Cu" "B.Cu") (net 6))
 (segment (start 58.16 31.9) (end 62.66 31.9) (width 0.3) (layer "B.Cu") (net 6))
 (segment (start 54.16 27.9) (end 58.16 31.9) (width 0.3) (layer "B.Cu") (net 6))
 (segment (start 68.5123 31.9) (end 68.5123 32.0477) (width 0.2) (layer "F.Cu") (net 1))
 (segment (start 68.5123 32.0477) (end 68.3646 32.1954) (width 0.2) (layer "F.Cu") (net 1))
 (segment (start 68.636 29.4) (end 68.636 31.7763) (width 0.3) (layer "F.Cu") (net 1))
 (segment (start 68.636 31.7763) (end 68.5123 31.9) (width 0.2) (layer "F.Cu") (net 1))
 (segment (start 68.3646 32.1954) (end 68.3646 34.4) (width 0.3) (layer "F.Cu") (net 1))
 (segment (start 68.5123 29.0477) (end 68.66 28.9) (width 0.2) (layer "F.Cu") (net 1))
 (segment (start 50.210001 40.535) (end 49.760001 40.985) (width 0.3) (layer "F.Cu") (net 3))
 (segment (start 49.760001 42.100001) (end 50.115 42.455) (width 0.3) (layer "F.Cu") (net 3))
 (segment (start 71.684 33.727607) (end 65.8538 39.557807) (width 0.3) (layer "F.Cu") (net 3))
 (segment (start 61.6125 39.7062) (end 61.760893 39.557807) (width 0.3) (layer "F.Cu") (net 3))
 (segment (start 50.115 42.455) (end 58.8637 42.455) (width 0.3) (layer "F.Cu") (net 3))
 (segment (start 71.684 29.4) (end 71.684 33.727607) (width 0.3) (layer "F.Cu") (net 3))
 (segment (start 61.760893 39.557807) (end 65.8538 39.557807) (width 0.3) (layer "F.Cu") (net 3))
 (segment (start 49.760001 40.985) (end 49.760001 42.100001) (width 0.3) (layer "F.Cu") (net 3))
 (segment (start 58.8637 42.455) (end 61.6125 39.7062) (width 0.3) (layer "F.Cu") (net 3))
 (segment (start 51.185 40.535) (end 50.210001 40.535) (width 0.3) (layer "F.Cu") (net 3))
 (segment (start 55.88 26.81) (end 58.97 29.9) (width 0.3) (layer "F.Cu") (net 8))
 (segment (start 55.88 25.4) (end 55.88 26.81) (width 0.3) (layer "F.Cu") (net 8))
 (segment (start 61.8 41) (end 60.7 42.1) (width 1) (layer "F.Cu") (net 4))
 (segment (start 66.06 41) (end 61.8 41) (width 1) (layer "F.Cu") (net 4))
 (via (at 66.06 41) (size 2) (drill 0.6) (layers "F.Cu" "B.Cu") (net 4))
 (segment (start 71.76 33.3) (end 66.06 39) (width 1) (layer "B.Cu") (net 4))
 (segment (start 65.1 27) (end 70.974214 27) (width 1) (layer "B.Cu") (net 4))
 (segment (start 65.1 27) (end 63.5 25.4) (width 1) (layer "B.Cu") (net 4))
 (segment (start 66.06 39) (end 66.06 41) (width 1) (layer "B.Cu") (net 4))
 (segment (start 71.76 27.785786) (end 71.76 33.3) (width 1) (layer "B.Cu") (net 4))
 (segment (start 70.974214 27) (end 71.76 27.785786) (width 1) (layer "B.Cu") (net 4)))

